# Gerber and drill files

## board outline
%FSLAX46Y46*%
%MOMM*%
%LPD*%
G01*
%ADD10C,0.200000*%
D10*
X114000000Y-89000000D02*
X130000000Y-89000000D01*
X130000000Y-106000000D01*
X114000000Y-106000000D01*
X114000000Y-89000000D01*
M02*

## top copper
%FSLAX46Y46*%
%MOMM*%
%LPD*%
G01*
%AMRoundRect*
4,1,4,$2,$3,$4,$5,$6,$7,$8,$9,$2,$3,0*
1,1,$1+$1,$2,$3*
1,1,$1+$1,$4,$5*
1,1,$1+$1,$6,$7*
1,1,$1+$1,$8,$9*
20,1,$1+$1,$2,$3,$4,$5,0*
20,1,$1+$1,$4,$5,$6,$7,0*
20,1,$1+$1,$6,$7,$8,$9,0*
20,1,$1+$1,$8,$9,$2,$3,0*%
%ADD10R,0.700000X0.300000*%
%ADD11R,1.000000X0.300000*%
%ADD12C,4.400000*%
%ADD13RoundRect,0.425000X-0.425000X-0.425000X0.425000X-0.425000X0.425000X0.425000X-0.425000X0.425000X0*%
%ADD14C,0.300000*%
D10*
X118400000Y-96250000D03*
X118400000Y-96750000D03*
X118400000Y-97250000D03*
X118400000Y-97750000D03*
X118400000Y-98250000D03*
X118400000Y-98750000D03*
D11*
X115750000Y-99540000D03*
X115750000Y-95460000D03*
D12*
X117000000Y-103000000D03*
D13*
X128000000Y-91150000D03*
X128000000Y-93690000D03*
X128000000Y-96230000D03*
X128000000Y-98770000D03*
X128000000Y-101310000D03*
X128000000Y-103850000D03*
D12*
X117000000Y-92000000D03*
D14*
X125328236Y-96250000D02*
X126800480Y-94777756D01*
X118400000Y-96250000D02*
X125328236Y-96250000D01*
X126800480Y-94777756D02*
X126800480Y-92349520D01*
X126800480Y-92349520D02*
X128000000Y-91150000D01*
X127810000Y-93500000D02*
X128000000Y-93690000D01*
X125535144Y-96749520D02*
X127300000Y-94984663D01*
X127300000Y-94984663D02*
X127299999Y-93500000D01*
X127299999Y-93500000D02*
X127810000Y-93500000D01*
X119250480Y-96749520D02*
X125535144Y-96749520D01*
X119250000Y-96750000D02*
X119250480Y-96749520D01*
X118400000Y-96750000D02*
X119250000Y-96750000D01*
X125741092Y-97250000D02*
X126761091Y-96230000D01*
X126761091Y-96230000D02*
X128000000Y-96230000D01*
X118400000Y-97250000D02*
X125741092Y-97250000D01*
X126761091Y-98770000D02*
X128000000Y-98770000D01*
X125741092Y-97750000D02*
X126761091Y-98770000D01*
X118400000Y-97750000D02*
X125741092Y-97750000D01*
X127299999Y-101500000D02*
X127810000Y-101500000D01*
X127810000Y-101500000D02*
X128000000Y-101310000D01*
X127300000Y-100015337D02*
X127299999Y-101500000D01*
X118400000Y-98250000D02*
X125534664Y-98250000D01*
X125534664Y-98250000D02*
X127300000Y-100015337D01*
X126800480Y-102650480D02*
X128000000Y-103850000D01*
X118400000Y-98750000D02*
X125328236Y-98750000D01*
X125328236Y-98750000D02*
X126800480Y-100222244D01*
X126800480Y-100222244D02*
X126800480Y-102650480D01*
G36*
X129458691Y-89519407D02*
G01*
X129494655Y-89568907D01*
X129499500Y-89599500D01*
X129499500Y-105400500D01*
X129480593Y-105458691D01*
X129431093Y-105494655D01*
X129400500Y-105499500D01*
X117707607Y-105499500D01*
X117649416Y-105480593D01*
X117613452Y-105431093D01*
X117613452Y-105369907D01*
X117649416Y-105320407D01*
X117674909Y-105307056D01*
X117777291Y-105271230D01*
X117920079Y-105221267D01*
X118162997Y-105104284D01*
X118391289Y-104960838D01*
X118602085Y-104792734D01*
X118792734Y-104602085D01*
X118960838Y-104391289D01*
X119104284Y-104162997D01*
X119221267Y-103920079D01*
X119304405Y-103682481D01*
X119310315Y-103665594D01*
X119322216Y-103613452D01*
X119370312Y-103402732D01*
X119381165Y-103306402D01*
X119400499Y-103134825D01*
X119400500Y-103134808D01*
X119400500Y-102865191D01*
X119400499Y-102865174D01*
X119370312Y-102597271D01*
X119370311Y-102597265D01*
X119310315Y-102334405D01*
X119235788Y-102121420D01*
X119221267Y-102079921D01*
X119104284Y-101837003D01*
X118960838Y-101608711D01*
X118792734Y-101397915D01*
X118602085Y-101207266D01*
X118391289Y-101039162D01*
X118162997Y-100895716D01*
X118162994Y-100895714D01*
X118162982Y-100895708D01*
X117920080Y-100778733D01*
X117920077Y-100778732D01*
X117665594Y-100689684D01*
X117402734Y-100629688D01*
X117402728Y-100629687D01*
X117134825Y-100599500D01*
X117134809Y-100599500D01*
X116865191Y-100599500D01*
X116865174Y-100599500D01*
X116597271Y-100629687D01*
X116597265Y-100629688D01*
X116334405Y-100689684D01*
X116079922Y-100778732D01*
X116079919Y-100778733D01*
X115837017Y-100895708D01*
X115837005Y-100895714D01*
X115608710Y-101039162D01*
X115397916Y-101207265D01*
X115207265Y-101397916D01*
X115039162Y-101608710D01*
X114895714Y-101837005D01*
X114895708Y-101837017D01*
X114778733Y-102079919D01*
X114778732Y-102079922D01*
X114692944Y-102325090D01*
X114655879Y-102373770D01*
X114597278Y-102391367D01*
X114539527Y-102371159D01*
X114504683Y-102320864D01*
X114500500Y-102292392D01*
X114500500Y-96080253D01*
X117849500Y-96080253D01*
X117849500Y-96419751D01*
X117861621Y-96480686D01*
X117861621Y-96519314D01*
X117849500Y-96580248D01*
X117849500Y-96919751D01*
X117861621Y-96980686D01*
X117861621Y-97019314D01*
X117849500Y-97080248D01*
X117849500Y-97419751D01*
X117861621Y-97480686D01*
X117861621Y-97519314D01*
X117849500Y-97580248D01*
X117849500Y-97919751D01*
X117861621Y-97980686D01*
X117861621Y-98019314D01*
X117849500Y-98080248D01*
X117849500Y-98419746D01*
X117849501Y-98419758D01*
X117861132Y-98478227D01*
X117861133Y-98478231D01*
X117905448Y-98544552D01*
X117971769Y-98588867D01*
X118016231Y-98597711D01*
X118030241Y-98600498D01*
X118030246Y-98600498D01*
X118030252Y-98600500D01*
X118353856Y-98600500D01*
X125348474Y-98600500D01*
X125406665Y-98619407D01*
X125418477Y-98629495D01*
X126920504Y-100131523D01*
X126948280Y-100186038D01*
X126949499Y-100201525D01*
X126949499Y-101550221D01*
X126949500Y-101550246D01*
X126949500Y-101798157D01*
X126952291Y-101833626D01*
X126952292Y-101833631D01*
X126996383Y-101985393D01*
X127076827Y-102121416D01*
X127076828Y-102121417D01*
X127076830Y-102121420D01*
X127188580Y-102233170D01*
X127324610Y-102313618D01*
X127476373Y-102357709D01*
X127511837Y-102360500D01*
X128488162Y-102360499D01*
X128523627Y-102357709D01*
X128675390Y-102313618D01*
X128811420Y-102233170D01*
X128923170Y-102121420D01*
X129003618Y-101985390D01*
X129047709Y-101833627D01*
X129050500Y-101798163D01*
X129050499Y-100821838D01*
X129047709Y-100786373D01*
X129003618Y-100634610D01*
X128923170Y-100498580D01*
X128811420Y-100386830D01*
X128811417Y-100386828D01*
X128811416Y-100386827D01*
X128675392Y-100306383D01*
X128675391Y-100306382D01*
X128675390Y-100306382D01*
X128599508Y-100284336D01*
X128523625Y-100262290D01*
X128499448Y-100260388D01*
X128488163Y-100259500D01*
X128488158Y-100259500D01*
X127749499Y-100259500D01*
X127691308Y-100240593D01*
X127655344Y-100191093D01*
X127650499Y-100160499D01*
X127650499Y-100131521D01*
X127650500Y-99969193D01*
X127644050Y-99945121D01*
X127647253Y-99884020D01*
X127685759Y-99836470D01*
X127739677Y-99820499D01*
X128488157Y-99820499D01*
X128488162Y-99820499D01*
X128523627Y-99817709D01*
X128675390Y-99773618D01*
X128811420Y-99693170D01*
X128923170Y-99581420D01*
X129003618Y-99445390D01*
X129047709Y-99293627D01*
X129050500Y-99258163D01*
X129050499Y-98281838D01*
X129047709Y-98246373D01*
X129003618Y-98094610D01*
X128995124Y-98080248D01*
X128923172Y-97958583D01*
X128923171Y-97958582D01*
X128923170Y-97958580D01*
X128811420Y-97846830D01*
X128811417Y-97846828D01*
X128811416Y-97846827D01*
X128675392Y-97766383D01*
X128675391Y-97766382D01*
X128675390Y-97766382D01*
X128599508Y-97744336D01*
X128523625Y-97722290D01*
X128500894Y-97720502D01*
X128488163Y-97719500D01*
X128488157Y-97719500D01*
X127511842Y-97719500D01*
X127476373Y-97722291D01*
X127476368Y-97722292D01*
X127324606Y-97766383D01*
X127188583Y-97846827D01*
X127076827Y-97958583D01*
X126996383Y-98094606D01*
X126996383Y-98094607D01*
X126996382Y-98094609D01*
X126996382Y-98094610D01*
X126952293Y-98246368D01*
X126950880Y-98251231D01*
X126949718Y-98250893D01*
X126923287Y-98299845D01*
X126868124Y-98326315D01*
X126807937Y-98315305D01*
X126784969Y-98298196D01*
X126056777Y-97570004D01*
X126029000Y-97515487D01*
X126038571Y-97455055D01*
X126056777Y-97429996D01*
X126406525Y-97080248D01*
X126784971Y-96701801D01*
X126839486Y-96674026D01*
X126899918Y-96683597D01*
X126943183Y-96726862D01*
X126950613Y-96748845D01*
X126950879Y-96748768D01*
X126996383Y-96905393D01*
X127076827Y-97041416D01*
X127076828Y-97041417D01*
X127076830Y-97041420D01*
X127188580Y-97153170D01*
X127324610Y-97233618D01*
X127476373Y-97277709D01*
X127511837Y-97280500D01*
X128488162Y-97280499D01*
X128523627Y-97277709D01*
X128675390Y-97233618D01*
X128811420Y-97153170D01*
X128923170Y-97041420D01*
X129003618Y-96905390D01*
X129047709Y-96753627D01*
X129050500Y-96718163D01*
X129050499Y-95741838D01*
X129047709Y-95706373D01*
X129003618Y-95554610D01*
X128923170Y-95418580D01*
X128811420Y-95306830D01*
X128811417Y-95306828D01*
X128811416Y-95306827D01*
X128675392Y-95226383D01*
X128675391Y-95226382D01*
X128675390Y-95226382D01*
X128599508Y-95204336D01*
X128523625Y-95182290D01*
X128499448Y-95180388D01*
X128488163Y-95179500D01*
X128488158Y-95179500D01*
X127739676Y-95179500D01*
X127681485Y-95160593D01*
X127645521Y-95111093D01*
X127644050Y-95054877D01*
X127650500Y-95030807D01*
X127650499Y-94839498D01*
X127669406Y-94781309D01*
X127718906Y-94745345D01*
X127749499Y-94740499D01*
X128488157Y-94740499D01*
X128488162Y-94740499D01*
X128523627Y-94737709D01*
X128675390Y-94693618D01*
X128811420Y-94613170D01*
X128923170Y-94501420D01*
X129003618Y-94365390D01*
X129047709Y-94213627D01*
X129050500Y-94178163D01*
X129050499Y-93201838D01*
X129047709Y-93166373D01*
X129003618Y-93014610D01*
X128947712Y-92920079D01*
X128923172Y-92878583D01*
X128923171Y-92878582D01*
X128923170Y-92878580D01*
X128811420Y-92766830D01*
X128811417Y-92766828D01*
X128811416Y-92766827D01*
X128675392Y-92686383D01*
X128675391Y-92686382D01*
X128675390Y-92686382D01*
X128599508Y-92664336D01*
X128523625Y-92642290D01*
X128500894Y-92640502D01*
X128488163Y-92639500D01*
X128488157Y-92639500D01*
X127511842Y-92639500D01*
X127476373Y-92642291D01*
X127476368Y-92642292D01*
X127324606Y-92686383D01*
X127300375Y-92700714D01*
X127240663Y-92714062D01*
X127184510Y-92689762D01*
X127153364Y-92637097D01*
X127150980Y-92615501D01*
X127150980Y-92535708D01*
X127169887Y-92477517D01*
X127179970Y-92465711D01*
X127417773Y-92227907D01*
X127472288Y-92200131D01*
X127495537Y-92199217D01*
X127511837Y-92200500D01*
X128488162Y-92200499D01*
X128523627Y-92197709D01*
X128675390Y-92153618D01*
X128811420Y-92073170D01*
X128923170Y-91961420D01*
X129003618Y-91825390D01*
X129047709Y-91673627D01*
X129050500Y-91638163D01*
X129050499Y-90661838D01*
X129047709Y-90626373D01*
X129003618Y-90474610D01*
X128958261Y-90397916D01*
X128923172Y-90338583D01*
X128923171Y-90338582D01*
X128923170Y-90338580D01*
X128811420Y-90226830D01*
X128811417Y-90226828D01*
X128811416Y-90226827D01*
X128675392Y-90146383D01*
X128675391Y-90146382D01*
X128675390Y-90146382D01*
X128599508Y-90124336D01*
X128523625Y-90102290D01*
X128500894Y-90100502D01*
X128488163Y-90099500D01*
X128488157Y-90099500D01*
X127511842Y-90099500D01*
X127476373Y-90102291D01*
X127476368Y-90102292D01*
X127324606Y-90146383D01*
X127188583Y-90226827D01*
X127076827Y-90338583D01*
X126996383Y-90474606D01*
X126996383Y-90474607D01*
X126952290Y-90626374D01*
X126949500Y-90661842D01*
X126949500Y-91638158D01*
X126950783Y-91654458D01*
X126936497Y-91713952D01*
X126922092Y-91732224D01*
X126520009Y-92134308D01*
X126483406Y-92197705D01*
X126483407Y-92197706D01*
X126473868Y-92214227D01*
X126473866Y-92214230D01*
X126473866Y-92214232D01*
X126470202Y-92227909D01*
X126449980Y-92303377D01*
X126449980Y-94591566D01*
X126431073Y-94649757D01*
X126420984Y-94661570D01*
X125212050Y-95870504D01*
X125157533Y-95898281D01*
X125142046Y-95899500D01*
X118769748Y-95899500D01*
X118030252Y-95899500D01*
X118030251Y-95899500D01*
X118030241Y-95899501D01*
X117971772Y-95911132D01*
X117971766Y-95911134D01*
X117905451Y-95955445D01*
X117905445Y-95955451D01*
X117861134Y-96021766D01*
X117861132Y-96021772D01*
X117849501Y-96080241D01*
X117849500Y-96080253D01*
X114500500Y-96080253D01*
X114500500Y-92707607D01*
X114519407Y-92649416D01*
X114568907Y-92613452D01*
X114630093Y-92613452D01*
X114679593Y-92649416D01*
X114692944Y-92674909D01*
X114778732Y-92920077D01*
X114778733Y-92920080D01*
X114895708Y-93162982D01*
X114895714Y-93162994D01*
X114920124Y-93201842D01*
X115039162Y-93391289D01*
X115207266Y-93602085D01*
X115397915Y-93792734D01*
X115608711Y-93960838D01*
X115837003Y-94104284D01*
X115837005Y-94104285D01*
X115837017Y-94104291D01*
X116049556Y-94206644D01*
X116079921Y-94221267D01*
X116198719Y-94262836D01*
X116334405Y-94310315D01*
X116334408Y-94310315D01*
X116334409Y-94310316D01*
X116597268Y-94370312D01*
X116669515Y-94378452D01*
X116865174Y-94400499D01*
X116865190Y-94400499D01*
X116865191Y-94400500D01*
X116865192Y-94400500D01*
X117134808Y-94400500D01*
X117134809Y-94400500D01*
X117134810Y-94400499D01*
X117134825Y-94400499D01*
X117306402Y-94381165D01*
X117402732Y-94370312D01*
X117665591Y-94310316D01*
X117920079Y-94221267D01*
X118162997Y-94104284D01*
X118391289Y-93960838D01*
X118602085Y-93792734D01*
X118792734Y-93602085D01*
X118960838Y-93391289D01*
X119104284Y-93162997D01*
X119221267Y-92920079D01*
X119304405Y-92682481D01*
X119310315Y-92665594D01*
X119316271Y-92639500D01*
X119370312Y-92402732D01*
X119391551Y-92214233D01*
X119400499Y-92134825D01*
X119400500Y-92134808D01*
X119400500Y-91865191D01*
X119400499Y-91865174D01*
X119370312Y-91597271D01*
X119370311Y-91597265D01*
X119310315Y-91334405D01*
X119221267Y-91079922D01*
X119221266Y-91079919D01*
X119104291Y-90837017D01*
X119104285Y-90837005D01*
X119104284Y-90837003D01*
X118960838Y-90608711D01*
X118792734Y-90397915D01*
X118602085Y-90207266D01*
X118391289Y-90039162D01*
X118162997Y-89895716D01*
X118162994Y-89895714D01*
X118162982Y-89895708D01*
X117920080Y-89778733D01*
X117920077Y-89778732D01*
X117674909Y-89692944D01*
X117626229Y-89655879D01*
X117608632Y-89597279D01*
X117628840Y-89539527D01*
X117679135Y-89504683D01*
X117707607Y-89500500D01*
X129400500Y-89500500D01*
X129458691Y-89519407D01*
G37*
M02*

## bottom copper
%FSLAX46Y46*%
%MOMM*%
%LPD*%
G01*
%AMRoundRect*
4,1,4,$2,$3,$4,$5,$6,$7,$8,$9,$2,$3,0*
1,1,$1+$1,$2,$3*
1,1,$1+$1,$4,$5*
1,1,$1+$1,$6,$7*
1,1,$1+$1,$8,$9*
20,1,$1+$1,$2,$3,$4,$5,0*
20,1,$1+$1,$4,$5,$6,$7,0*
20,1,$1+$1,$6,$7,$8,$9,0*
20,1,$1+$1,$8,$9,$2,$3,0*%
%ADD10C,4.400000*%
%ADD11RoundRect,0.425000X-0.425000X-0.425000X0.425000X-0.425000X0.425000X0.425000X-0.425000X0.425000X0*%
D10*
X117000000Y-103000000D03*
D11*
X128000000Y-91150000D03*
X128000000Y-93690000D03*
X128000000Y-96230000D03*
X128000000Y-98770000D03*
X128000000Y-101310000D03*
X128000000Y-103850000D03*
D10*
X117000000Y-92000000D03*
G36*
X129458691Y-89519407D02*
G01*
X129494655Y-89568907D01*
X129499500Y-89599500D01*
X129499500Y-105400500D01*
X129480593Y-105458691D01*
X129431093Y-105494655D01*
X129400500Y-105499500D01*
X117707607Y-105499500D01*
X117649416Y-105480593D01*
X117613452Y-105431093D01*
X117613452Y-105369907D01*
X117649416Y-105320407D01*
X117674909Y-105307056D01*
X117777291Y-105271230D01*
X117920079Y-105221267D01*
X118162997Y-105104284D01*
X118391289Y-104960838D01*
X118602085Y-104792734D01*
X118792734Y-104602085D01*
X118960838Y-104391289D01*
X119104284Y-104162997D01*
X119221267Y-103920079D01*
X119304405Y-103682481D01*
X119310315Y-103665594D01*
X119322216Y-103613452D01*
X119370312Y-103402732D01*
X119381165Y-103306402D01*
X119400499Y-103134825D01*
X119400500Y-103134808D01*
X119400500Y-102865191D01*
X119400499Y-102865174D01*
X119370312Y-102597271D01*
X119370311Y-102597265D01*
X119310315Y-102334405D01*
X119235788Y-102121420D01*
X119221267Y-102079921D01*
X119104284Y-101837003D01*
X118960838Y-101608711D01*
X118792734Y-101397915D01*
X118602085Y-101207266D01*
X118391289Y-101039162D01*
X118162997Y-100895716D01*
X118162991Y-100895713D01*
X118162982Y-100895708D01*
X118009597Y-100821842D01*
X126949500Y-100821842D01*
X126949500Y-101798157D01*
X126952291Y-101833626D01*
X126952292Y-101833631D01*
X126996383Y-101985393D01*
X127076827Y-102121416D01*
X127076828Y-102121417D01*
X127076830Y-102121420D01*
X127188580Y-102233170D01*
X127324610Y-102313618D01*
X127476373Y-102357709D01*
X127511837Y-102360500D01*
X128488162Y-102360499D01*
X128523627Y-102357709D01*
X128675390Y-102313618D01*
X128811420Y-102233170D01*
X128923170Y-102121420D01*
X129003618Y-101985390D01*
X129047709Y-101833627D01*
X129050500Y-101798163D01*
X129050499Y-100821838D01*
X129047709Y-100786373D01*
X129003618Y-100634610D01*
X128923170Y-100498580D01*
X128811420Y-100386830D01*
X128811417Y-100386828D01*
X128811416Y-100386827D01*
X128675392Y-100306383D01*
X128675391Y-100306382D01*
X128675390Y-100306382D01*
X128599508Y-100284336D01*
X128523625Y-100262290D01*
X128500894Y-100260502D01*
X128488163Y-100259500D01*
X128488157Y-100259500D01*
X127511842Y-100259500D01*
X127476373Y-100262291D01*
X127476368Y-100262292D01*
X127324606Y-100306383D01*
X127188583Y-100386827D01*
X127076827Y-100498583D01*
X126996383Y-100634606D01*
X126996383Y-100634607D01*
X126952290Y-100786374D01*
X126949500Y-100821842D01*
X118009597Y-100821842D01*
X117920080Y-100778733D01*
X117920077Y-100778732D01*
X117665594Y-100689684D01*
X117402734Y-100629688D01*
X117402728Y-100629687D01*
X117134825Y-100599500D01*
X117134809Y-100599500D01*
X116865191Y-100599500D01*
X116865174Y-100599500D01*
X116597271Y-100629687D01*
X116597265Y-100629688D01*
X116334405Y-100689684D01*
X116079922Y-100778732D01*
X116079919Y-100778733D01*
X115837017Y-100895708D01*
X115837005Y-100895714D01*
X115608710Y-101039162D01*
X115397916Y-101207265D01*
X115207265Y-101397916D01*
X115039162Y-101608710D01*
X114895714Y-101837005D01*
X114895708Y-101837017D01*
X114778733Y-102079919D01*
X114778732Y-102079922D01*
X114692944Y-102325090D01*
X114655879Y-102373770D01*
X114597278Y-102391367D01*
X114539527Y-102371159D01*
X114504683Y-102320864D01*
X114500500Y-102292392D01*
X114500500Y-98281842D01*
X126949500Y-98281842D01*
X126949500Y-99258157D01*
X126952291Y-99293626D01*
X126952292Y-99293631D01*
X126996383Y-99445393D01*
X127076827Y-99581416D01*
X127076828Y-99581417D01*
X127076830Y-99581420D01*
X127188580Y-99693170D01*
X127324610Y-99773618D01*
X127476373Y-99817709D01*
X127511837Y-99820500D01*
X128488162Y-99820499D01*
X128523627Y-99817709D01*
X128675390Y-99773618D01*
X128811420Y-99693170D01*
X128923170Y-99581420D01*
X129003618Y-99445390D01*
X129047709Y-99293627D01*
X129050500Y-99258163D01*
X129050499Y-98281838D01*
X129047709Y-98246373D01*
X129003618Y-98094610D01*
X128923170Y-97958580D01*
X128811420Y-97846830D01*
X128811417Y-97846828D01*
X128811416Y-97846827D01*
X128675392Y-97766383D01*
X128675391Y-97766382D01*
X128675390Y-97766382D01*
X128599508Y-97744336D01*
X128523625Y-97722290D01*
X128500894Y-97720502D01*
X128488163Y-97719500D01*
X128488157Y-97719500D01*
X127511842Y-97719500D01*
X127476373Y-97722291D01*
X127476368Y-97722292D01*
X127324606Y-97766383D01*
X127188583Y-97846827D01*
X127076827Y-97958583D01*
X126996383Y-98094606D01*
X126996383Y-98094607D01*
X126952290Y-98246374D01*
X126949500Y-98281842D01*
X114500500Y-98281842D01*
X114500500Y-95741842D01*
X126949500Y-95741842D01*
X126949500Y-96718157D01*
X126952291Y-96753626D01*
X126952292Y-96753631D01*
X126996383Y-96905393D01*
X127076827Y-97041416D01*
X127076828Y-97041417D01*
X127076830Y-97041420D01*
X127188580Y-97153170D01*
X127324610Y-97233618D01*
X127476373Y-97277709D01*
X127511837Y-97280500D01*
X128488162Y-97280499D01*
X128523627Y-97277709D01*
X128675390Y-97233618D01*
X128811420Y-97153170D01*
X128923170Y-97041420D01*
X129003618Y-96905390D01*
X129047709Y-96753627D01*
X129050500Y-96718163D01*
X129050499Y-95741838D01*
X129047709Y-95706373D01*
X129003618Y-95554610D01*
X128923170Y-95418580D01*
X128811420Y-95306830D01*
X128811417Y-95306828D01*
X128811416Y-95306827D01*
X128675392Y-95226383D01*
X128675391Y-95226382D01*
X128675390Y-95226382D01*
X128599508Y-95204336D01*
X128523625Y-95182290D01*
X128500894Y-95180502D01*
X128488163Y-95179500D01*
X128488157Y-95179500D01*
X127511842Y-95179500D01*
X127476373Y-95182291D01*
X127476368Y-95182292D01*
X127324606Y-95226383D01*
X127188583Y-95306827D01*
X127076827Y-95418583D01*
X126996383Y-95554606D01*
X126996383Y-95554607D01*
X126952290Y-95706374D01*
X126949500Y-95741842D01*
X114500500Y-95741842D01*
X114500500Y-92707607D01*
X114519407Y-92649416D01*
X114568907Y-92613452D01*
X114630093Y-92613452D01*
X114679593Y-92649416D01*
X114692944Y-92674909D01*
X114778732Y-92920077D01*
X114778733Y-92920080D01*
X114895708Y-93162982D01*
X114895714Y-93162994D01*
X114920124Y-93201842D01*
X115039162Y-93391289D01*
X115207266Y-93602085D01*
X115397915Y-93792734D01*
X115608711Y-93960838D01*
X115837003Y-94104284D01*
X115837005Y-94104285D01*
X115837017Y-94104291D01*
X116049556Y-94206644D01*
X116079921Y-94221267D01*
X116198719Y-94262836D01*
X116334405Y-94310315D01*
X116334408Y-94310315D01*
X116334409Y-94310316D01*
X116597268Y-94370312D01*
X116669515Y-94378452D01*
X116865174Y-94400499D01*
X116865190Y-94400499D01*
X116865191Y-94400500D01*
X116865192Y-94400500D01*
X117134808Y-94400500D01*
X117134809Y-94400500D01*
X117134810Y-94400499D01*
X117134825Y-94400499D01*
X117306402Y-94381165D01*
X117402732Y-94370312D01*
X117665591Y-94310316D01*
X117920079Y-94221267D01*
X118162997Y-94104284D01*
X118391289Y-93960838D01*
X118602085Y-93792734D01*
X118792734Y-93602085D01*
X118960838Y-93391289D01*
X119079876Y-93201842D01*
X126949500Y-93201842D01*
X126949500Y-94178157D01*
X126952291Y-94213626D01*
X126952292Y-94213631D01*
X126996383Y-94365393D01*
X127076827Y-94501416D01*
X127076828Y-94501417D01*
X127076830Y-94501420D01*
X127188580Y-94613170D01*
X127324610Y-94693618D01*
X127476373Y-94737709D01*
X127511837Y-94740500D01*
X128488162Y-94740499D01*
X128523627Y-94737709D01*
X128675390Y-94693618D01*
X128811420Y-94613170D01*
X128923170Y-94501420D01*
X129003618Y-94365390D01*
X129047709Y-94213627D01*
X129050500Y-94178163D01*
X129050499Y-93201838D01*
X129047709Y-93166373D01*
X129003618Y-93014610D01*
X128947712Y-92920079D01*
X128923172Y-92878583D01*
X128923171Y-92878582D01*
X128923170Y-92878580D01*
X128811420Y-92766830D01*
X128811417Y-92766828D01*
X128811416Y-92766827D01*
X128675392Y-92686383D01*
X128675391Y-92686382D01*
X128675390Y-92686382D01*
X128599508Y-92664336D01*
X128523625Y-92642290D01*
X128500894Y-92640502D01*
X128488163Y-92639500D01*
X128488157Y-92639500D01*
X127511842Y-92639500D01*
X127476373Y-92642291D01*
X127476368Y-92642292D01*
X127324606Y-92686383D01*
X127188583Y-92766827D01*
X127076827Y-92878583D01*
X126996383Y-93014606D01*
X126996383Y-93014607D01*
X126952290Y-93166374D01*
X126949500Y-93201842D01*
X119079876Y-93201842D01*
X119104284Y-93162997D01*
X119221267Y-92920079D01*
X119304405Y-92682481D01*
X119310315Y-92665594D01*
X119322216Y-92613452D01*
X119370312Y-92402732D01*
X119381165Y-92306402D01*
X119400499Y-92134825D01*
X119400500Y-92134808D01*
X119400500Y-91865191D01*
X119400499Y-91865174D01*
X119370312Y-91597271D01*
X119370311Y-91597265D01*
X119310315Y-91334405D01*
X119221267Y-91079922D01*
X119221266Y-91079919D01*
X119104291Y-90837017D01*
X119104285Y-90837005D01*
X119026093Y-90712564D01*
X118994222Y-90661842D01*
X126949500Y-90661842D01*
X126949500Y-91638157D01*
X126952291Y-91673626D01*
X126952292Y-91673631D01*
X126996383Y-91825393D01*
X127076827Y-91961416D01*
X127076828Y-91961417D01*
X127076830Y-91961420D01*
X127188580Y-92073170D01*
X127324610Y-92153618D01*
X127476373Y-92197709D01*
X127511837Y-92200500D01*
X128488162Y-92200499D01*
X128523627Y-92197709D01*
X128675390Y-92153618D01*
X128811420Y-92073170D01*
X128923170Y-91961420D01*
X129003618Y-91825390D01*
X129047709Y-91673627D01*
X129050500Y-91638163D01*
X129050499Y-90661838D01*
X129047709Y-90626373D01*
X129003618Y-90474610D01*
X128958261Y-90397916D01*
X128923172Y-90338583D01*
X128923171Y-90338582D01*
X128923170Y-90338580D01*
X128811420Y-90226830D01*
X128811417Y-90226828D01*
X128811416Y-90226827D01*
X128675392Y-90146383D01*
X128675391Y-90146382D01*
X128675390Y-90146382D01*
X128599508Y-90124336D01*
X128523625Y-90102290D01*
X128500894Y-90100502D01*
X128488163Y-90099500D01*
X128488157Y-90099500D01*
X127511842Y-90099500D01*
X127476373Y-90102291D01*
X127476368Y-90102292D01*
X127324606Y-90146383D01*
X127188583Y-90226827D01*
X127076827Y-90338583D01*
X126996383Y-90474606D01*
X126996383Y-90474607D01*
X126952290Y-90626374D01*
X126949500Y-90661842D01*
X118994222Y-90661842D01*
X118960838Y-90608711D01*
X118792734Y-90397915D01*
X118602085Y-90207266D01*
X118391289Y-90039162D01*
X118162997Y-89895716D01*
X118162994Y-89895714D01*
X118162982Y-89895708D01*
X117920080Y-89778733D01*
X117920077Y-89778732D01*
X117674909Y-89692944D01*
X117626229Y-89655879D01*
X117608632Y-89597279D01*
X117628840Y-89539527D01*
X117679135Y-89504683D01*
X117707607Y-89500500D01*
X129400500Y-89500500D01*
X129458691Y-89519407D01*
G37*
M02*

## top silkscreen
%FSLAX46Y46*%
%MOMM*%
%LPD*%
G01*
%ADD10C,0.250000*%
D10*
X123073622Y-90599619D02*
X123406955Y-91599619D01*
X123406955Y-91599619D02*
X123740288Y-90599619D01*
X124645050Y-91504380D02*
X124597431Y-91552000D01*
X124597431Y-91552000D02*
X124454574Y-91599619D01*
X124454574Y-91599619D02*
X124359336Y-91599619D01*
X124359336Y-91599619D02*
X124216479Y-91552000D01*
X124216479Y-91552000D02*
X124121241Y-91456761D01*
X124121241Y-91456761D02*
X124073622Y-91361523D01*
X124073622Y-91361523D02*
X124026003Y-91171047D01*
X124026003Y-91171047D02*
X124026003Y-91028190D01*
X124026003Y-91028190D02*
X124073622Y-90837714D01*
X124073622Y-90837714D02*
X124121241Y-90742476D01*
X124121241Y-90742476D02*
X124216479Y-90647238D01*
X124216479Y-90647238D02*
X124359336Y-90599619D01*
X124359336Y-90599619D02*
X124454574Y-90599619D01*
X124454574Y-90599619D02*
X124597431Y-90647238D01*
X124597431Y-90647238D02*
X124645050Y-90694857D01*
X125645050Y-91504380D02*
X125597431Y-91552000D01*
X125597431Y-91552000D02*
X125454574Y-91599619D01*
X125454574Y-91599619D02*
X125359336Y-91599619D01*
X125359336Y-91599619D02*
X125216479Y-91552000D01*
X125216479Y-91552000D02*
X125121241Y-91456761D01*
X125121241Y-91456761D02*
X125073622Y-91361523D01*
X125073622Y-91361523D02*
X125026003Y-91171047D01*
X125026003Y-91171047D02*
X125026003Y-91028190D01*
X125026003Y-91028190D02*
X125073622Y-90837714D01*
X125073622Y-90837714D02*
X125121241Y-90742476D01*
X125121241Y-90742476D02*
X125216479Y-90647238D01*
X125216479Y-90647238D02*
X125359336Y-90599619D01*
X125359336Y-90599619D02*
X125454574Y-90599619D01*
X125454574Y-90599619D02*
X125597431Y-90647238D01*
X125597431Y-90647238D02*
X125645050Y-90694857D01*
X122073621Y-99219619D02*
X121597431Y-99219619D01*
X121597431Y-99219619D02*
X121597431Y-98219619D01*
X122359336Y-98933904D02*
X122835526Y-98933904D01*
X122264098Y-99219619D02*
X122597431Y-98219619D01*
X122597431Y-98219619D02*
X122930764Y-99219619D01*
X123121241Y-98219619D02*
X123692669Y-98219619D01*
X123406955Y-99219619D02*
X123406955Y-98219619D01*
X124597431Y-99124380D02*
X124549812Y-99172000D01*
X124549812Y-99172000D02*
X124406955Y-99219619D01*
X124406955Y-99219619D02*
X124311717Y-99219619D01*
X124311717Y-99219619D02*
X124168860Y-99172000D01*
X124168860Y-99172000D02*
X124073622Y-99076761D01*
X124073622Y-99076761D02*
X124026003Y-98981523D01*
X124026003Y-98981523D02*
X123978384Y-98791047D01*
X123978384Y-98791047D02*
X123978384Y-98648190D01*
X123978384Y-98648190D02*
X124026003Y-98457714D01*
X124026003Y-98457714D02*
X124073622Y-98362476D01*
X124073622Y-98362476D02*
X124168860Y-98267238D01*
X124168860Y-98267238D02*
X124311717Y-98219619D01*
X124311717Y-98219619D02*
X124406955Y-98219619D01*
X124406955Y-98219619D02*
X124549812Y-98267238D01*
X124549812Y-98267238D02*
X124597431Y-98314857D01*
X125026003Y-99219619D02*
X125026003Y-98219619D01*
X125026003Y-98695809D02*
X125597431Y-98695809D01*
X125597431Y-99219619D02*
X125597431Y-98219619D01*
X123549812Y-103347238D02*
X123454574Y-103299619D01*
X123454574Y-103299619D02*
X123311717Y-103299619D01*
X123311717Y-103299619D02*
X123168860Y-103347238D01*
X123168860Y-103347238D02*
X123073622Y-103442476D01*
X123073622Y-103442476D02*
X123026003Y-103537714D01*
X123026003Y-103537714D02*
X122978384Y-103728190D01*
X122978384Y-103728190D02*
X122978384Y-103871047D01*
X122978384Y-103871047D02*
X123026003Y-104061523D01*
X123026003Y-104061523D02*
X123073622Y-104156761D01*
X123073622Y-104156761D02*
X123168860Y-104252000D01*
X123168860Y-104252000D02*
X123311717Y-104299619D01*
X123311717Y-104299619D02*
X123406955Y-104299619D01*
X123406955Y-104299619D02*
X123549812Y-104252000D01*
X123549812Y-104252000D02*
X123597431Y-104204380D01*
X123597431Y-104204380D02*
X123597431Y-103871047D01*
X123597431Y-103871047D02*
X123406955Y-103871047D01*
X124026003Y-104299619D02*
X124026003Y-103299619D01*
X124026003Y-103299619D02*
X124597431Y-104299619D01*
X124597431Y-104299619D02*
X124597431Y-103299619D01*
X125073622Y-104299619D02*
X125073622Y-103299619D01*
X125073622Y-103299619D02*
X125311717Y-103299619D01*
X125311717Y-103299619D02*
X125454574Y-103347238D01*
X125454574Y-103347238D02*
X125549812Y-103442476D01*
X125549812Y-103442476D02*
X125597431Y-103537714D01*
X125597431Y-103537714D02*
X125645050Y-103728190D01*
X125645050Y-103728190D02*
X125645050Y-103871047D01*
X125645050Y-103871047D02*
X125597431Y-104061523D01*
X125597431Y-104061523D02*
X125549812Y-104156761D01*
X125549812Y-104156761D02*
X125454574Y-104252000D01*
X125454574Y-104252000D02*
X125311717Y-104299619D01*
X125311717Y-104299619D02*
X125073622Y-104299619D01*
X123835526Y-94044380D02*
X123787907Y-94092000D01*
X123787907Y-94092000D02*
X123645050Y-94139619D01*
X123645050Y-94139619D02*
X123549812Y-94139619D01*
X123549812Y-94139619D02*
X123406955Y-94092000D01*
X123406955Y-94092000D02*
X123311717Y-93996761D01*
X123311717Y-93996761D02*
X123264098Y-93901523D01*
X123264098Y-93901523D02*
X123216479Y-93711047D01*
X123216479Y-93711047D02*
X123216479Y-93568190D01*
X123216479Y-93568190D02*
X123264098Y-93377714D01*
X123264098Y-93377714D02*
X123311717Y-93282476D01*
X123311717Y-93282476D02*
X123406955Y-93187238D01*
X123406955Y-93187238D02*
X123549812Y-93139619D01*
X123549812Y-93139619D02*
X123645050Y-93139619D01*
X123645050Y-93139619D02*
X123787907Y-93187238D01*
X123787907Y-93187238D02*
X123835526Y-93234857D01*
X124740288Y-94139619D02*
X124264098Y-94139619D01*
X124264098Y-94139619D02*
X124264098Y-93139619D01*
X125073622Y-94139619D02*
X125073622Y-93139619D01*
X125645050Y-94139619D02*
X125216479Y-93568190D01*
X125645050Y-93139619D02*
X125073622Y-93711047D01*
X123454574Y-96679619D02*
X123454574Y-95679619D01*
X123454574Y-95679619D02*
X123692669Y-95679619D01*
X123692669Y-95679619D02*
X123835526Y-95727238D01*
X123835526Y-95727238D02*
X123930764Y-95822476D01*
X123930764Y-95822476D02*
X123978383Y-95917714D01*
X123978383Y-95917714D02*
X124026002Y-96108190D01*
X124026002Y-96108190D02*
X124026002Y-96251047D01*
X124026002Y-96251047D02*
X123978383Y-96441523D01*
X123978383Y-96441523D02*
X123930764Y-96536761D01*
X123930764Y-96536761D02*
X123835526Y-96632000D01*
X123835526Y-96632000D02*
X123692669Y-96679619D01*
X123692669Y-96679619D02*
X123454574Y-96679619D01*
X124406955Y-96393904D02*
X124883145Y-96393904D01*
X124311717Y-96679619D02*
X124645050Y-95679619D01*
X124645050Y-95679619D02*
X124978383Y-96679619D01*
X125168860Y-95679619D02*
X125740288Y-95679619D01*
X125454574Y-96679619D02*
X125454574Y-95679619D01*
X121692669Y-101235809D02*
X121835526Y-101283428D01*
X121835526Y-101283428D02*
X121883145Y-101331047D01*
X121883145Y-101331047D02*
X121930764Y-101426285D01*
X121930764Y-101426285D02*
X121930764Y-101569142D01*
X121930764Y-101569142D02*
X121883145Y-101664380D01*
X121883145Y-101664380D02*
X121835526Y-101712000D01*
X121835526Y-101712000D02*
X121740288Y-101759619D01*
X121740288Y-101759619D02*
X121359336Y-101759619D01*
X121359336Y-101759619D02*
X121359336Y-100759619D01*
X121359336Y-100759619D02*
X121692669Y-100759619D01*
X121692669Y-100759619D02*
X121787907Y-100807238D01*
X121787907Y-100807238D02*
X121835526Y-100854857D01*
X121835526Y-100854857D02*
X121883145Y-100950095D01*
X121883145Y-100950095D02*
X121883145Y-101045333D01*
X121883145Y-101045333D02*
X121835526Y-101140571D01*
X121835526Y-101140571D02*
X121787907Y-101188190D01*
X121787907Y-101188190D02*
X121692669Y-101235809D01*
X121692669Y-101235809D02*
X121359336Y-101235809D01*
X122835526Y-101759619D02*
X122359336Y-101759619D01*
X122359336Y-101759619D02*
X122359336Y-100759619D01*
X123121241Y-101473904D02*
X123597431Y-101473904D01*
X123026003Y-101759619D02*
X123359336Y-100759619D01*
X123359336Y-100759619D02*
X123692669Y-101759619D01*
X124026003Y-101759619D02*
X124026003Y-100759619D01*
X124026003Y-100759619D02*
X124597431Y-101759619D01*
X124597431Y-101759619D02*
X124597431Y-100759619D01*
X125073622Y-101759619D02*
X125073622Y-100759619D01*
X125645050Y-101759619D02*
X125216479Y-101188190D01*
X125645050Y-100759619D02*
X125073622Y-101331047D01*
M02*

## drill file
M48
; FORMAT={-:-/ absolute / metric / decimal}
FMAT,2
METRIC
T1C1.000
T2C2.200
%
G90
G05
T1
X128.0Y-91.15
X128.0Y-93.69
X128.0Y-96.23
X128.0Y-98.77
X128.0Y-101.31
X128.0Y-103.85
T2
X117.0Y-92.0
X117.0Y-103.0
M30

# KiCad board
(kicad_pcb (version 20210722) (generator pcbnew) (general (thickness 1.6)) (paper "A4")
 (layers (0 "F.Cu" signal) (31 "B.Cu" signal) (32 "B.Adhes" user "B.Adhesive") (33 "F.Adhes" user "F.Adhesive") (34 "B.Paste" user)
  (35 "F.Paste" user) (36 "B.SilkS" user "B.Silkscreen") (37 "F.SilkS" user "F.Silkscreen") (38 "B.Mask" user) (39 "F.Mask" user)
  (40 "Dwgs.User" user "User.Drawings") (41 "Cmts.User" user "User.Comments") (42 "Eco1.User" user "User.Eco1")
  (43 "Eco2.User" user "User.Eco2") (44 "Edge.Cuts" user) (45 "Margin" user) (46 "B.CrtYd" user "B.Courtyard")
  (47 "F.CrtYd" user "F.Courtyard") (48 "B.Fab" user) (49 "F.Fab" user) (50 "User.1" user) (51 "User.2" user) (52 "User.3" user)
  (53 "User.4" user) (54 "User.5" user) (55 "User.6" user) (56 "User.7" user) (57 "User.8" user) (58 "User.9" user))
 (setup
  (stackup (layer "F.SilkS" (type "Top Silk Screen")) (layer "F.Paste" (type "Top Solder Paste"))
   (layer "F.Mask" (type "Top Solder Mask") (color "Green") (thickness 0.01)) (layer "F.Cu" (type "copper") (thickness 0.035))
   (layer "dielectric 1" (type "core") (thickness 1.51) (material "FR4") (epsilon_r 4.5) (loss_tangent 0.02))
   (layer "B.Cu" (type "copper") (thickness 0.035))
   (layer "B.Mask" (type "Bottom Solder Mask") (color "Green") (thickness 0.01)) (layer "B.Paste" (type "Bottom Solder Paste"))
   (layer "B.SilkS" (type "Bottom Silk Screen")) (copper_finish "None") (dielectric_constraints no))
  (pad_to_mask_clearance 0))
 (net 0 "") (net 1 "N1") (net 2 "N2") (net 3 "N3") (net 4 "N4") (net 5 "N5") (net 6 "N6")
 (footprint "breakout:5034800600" (layer "F.Cu") (at 117 97.5 -90)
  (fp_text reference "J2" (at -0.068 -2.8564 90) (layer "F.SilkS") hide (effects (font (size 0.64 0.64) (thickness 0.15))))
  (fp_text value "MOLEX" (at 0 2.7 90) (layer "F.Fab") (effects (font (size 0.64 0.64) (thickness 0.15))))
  (pad "1" smd rect locked (at -1.25 -1.4 270) (size 0.3 0.7) (layers "F.Cu" "F.Paste" "F.Mask") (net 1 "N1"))
  (pad "2" smd rect locked (at -0.75 -1.4 270) (size 0.3 0.7) (layers "F.Cu" "F.Paste" "F.Mask") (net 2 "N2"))
  (pad "3" smd rect locked (at -0.25 -1.4 270) (size 0.3 0.7) (layers "F.Cu" "F.Paste" "F.Mask") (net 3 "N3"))
  (pad "4" smd rect locked (at 0.25 -1.4 270) (size 0.3 0.7) (layers "F.Cu" "F.Paste" "F.Mask") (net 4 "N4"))
  (pad "5" smd rect locked (at 0.75 -1.4 270) (size 0.3 0.7) (layers "F.Cu" "F.Paste" "F.Mask") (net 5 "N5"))
  (pad "6" smd rect locked (at 1.25 -1.4 270) (size 0.3 0.7) (layers "F.Cu" "F.Paste" "F.Mask") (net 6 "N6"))
  (pad "SH" smd rect locked (at 2.04 1.25 270) (size 0.3 1) (layers "F.Cu" "F.Paste" "F.Mask") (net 6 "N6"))
  (pad "SH" smd rect locked (at -2.04 1.25 270) (size 0.3 1) (layers "F.Cu" "F.Paste" "F.Mask") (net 6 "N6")))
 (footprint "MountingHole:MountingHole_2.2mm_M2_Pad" (layer "F.Cu") (at 117 103)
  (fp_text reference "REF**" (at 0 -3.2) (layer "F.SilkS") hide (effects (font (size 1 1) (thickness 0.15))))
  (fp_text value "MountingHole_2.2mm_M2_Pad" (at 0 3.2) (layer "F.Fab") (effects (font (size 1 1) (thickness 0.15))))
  (pad "1" thru_hole circle locked (at 0 0) (size 4.4 4.4) (drill 2.2) (layers *.Cu *.Mask)))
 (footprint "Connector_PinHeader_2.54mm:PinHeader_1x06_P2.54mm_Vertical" (layer "F.Cu") (at 128 91.15)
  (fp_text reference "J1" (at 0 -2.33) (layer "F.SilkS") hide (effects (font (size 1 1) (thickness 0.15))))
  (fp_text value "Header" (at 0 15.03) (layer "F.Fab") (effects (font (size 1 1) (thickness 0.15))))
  (pad "1" thru_hole roundrect locked (at 0 0) (size 1.7 1.7) (drill 1) (layers *.Cu *.Mask) (roundrect_rratio 0.25) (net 1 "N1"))
  (pad "2" thru_hole roundrect locked (at 0 2.54) (size 1.7 1.7) (drill 1) (layers *.Cu *.Mask) (roundrect_rratio 0.25) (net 2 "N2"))
  (pad "3" thru_hole roundrect locked (at 0 5.08) (size 1.7 1.7) (drill 1) (layers *.Cu *.Mask) (roundrect_rratio 0.25) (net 3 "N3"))
  (pad "4" thru_hole roundrect locked (at 0 7.62) (size 1.7 1.7) (drill 1) (layers *.Cu *.Mask) (roundrect_rratio 0.25) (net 4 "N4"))
  (pad "5" thru_hole roundrect locked (at 0 10.16) (size 1.7 1.7) (drill 1) (layers *.Cu *.Mask) (roundrect_rratio 0.25) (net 5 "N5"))
  (pad "6" thru_hole roundrect locked (at 0 12.7) (size 1.7 1.7) (drill 1) (layers *.Cu *.Mask) (roundrect_rratio 0.25) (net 6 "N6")))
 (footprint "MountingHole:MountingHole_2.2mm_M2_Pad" (layer "F.Cu") (at 117 92)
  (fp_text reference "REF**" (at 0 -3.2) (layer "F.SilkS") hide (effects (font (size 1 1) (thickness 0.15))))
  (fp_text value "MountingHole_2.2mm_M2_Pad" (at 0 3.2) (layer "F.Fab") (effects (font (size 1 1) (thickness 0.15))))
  (pad "1" thru_hole circle locked (at 0 0) (size 4.4 4.4) (drill 2.2) (layers *.Cu *.Mask)))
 (gr_rect (start 114 89) (end 130 106) (layer "Edge.Cuts") (width 0.2) (fill none))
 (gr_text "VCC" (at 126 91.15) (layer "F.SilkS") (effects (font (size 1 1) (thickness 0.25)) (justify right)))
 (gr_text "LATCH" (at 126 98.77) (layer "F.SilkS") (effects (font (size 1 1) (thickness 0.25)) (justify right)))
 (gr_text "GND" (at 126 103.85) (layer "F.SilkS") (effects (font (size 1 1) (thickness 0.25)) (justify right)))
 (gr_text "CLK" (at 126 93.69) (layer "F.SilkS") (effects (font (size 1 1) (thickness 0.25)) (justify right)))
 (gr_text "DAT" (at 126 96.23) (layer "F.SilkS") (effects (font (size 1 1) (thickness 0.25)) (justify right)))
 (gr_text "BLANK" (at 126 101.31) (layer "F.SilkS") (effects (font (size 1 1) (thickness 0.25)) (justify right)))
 (segment (start 125.328236 96.25) (end 126.80048 94.777756) (width 0.3) (layer "F.Cu") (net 1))
 (segment (start 118.4 96.25) (end 125.328236 96.25) (width 0.3) (layer "F.Cu") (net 1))
 (segment (start 126.80048 94.777756) (end 126.80048 92.34952) (width 0.3) (layer "F.Cu") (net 1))
 (segment (start 126.80048 92.34952) (end 128 91.15) (width 0.3) (layer "F.Cu") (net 1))
 (segment (start 127.81 93.5) (end 128 93.69) (width 0.3) (layer "F.Cu") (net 2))
 (segment (start 125.535144 96.74952) (end 127.3 94.984663) (width 0.3) (layer "F.Cu") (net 2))
 (segment (start 127.3 94.984663) (end 127.299999 93.5) (width 0.3) (layer "F.Cu") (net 2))
 (segment (start 127.299999 93.5) (end 127.81 93.5) (width 0.3) (layer "F.Cu") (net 2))
 (segment (start 119.25048 96.74952) (end 125.535144 96.74952) (width 0.3) (layer "F.Cu") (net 2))
 (segment (start 119.25 96.75) (end 119.25048 96.74952) (width 0.3) (layer "F.Cu") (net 2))
 (segment (start 118.4 96.75) (end 119.25 96.75) (width 0.3) (layer "F.Cu") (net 2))
 (segment (start 125.741092 97.25) (end 126.761091 96.23) (width 0.3) (layer "F.Cu") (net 3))
 (segment (start 126.761091 96.23) (end 128 96.23) (width 0.3) (layer "F.Cu") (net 3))
 (segment (start 118.4 97.25) (end 125.741092 97.25) (width 0.3) (layer "F.Cu") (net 3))
 (segment (start 126.761091 98.77) (end 128 98.77) (width 0.3) (layer "F.Cu") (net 4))
 (segment (start 125.741092 97.75) (end 126.761091 98.77) (width 0.3) (layer "F.Cu") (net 4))
 (segment (start 118.4 97.75) (end 125.741092 97.75) (width 0.3) (layer "F.Cu") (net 4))
 (segment (start 127.299999 101.5) (end 127.81 101.5) (width 0.3) (layer "F.Cu") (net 5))
 (segment (start 127.81 101.5) (end 128 101.31) (width 0.3) (layer "F.Cu") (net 5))
 (segment (start 127.3 100.015337) (end 127.299999 101.5) (width 0.3) (layer "F.Cu") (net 5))
 (segment (start 118.4 98.25) (end 125.534664 98.25) (width 0.3) (layer "F.Cu") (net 5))
 (segment (start 125.534664 98.25) (end 127.3 100.015337) (width 0.3) (layer "F.Cu") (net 5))
 (segment (start 126.80048 102.65048) (end 128 103.85) (width 0.3) (layer "F.Cu") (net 6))
 (segment (start 118.4 98.75) (end 125.328236 98.75) (width 0.3) (layer "F.Cu") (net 6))
 (segment (start 125.328236 98.75) (end 126.80048 100.222244) (width 0.3) (layer "F.Cu") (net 6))
 (segment (start 126.80048 100.222244) (end 126.80048 102.65048) (width 0.3) (layer "F.Cu") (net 6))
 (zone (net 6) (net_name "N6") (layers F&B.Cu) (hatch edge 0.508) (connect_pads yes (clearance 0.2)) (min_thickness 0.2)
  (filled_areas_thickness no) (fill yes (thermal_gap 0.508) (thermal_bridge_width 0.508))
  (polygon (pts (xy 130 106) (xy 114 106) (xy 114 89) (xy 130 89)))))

